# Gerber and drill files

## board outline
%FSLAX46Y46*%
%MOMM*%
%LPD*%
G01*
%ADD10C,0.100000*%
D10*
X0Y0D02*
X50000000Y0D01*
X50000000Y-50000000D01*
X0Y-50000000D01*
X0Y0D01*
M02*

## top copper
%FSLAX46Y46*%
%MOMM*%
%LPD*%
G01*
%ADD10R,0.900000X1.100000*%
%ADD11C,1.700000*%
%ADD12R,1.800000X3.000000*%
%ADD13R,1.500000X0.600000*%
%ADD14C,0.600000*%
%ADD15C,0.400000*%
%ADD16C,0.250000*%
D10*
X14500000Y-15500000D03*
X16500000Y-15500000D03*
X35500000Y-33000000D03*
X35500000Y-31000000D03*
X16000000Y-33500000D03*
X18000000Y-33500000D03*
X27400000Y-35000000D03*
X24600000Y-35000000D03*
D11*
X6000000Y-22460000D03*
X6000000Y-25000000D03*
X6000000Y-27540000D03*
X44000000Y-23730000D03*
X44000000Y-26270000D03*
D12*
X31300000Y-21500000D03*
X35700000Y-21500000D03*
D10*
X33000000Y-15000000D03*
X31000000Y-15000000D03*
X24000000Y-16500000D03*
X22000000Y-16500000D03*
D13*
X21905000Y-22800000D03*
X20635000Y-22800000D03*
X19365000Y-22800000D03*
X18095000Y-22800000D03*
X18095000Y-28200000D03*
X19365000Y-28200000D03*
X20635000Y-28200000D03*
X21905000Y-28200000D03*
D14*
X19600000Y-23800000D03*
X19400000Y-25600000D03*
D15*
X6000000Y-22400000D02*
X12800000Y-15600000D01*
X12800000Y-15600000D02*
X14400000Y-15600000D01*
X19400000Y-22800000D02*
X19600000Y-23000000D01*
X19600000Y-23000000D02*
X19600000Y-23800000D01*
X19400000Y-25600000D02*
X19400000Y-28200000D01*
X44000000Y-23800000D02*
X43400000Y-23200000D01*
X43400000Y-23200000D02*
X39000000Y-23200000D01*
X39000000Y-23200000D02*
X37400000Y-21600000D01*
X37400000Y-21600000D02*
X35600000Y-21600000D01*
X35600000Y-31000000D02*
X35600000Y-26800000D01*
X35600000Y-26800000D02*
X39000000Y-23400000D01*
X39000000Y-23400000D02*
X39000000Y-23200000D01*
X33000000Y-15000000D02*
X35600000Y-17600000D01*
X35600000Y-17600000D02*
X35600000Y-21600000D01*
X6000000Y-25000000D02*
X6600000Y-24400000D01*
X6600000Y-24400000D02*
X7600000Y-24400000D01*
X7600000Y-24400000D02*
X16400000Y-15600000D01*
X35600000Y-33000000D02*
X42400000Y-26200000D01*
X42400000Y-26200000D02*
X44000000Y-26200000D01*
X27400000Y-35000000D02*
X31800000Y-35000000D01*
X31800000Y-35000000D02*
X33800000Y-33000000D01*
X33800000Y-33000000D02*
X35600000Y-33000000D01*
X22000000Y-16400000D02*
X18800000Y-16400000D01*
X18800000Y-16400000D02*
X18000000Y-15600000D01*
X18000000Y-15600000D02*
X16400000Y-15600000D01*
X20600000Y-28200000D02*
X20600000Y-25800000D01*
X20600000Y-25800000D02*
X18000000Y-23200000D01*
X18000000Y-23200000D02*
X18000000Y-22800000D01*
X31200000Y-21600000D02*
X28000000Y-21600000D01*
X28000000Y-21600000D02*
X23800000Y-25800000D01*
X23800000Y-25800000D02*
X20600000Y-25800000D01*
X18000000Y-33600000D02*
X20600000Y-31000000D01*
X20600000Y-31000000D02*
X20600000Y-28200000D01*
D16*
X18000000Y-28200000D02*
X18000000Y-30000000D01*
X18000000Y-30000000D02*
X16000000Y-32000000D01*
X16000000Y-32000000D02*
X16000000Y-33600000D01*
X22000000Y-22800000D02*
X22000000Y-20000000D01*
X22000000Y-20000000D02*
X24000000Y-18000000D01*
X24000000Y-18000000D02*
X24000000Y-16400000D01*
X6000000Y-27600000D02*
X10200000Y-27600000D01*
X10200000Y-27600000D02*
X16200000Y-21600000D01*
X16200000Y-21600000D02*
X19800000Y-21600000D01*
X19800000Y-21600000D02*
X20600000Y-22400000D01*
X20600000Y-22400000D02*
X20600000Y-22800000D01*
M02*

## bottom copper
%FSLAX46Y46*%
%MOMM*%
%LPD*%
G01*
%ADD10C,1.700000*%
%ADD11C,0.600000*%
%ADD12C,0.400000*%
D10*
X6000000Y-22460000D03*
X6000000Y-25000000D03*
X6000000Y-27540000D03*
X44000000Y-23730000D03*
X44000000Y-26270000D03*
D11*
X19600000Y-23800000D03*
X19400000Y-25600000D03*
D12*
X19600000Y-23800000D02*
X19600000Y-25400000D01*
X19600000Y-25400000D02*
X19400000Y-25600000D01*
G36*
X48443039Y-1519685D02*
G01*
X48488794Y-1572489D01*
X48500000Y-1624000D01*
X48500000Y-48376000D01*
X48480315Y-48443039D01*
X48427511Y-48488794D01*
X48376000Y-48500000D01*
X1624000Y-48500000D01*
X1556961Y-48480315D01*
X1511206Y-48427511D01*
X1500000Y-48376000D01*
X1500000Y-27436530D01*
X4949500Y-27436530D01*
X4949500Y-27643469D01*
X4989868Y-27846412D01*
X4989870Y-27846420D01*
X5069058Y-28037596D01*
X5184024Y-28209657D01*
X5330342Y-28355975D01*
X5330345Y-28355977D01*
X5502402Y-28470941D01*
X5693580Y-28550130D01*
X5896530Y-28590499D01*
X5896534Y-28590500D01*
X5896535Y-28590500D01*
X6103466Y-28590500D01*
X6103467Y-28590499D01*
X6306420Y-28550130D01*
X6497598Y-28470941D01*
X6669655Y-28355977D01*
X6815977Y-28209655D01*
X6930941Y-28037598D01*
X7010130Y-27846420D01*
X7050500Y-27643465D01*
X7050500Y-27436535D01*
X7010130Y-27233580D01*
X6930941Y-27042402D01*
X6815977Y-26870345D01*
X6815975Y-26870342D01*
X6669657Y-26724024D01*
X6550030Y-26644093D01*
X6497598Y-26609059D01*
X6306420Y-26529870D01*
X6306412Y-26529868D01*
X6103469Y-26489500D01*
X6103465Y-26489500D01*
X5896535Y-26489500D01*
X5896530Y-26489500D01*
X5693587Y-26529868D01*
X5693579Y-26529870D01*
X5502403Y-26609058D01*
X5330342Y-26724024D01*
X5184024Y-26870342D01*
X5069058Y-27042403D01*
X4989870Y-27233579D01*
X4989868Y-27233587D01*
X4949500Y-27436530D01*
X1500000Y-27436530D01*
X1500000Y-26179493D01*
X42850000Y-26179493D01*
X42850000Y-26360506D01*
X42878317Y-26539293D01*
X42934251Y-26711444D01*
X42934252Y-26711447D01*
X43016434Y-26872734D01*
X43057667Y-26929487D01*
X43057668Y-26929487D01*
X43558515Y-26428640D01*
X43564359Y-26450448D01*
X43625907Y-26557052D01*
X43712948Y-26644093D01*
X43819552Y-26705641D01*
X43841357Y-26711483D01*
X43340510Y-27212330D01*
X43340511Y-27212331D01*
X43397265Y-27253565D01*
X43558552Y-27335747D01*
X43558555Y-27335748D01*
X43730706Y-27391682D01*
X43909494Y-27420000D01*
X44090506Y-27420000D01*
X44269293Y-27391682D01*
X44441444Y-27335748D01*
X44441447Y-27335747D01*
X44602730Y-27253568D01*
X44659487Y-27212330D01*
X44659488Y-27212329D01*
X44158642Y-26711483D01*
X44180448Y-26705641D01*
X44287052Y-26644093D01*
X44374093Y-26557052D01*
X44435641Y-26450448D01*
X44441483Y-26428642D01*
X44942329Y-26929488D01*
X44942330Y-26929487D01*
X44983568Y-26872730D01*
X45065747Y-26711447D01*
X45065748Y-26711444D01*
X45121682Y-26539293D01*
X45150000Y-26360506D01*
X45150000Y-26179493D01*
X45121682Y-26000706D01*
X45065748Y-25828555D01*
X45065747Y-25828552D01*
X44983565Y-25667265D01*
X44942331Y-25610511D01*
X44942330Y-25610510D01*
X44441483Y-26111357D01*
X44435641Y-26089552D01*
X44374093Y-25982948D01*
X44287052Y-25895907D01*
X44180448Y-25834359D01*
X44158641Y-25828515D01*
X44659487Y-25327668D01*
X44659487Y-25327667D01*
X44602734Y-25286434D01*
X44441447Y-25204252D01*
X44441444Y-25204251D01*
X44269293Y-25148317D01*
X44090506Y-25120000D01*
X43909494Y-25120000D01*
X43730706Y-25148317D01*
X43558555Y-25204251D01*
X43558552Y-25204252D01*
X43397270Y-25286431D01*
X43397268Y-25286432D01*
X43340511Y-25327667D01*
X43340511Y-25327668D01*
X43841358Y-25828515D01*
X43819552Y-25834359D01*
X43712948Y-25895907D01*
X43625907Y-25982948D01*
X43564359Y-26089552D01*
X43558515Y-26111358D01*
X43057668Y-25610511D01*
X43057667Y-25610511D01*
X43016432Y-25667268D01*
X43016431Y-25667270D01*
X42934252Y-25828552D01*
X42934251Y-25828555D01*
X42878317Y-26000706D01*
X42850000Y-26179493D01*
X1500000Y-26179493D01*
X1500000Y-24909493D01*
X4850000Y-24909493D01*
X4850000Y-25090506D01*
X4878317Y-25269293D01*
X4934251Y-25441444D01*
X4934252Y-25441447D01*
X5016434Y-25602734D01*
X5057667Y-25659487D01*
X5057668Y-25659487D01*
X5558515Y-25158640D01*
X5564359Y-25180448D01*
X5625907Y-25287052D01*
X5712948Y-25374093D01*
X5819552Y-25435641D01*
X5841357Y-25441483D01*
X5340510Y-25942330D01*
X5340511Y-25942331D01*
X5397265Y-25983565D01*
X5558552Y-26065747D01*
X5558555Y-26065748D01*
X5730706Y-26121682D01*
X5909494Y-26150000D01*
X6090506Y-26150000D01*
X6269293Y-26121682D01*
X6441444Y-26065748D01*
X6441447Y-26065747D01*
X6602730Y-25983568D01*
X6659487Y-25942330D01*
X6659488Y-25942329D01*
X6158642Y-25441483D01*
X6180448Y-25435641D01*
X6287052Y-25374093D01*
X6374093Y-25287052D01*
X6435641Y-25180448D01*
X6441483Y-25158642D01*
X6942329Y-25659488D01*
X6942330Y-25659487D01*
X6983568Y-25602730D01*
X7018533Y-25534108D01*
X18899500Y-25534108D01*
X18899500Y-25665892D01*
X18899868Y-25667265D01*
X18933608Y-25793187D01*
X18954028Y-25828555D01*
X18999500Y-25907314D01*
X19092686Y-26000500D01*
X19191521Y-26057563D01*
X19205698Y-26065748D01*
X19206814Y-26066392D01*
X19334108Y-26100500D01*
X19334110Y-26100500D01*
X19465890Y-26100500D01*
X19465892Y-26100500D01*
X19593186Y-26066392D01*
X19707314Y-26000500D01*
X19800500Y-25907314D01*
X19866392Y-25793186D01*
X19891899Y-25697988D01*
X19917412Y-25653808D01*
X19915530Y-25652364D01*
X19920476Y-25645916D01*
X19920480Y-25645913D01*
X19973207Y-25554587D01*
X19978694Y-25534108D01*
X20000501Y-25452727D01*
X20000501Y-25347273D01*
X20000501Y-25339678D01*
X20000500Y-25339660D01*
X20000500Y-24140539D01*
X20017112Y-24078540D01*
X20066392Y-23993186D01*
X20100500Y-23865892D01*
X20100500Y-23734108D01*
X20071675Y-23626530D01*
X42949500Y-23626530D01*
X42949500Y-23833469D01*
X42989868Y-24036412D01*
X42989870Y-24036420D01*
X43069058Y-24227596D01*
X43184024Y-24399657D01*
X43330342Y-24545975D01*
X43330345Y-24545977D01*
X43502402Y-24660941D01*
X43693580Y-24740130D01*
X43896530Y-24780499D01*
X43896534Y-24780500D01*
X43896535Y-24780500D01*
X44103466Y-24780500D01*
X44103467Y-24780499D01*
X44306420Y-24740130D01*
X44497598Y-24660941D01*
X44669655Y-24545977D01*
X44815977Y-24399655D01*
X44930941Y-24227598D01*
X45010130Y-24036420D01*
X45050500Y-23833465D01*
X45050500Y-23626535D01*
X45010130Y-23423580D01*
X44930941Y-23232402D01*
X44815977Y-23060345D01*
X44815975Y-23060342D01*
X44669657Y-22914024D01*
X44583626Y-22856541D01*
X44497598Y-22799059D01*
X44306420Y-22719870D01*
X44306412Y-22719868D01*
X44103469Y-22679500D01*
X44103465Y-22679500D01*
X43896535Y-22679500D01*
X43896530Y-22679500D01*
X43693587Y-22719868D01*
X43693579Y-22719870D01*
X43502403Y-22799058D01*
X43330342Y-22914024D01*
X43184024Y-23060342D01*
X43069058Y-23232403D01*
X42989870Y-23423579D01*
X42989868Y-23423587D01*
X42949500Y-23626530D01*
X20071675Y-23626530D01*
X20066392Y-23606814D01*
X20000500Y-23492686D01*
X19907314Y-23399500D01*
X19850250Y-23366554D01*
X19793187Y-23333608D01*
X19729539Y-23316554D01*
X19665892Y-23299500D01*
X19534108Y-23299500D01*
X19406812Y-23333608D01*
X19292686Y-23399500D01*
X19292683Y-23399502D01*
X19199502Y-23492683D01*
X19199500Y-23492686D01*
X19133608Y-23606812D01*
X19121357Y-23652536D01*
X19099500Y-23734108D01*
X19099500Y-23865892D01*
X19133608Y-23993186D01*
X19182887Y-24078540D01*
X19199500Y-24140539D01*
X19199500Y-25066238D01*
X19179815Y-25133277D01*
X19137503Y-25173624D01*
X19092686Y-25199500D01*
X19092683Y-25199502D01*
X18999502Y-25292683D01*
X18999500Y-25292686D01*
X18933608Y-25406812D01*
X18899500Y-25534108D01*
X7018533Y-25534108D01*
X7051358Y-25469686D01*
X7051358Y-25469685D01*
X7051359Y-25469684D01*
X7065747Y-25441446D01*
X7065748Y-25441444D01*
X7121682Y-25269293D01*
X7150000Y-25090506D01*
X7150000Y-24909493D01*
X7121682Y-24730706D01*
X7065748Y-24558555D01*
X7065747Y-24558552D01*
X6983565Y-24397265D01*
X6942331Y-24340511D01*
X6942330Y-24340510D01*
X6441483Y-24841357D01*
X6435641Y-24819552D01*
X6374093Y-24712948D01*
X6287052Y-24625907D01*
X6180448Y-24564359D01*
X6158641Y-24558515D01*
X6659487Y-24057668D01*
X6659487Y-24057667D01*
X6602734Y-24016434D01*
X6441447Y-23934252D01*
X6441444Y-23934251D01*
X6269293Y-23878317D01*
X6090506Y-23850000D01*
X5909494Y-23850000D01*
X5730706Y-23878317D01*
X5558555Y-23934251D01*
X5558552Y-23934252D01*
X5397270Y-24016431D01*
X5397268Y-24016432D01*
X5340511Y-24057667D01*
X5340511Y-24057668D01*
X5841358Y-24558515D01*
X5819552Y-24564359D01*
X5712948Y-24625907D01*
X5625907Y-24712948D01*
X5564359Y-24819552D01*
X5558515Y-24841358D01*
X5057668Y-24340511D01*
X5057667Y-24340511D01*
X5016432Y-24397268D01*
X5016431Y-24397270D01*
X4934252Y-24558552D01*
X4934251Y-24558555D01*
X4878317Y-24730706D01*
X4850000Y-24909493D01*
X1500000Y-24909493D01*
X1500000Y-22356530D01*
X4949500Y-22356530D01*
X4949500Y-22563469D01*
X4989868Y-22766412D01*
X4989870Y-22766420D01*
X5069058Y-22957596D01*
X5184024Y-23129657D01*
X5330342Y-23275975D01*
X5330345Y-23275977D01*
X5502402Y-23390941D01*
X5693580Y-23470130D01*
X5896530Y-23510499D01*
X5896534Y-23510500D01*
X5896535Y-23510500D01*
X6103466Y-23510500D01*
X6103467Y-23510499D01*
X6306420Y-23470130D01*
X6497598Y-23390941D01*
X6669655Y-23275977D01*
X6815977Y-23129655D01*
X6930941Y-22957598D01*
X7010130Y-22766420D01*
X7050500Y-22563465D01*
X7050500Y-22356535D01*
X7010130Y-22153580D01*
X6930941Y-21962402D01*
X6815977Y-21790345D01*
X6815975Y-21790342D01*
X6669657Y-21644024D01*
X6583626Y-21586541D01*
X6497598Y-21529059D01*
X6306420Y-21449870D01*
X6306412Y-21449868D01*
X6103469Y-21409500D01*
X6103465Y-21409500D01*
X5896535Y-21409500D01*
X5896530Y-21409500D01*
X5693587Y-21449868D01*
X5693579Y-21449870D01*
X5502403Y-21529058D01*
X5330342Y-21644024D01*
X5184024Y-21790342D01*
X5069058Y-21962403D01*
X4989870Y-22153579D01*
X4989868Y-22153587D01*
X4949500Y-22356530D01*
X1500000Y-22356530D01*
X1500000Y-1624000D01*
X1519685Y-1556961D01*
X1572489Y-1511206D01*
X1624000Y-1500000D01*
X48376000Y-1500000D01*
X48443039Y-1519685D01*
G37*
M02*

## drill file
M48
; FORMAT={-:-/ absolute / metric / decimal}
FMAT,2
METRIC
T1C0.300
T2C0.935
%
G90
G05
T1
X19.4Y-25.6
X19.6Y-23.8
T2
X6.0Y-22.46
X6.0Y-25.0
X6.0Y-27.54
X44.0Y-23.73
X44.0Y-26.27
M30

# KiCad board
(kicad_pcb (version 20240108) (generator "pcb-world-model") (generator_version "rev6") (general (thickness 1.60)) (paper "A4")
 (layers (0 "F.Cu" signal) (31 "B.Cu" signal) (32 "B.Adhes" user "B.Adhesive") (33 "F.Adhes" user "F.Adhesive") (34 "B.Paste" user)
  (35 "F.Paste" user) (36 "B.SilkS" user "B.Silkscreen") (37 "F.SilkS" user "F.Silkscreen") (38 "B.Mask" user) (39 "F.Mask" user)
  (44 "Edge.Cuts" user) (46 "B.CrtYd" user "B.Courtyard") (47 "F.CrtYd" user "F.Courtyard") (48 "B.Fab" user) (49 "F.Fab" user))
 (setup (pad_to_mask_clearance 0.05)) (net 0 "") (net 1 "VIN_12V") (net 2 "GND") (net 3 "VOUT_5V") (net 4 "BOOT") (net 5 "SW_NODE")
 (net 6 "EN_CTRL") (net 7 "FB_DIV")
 (gr_rect (start 0.0 0.0) (end 50.0000 50.0000) (stroke (width 0.1) (type default)) (fill none) (layer "Edge.Cuts"))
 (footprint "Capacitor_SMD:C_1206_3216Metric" (layer "F.Cu") (at 15.5000 15.5000 0)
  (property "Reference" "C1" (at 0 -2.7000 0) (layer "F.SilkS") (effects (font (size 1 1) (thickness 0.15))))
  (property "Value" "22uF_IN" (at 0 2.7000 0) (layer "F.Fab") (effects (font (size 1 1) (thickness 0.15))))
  (pad "1" smd rect (at -1.0000 0.0000) (size 0.9000 1.1000) (layers "F.Cu" "F.Paste" "F.Mask") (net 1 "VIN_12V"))
  (pad "2" smd rect (at 1.0000 0.0000) (size 0.9000 1.1000) (layers "F.Cu" "F.Paste" "F.Mask") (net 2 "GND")))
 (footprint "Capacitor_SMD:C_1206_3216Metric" (layer "F.Cu") (at 35.5000 32.0000 90)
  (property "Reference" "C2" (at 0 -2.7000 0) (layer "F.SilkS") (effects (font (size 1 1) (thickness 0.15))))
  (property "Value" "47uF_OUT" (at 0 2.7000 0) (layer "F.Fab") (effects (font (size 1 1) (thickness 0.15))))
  (pad "1" smd rect (at -1.0000 0.0000) (size 0.9000 1.1000) (layers "F.Cu" "F.Paste" "F.Mask") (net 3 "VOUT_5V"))
  (pad "2" smd rect (at 1.0000 0.0000) (size 0.9000 1.1000) (layers "F.Cu" "F.Paste" "F.Mask") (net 2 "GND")))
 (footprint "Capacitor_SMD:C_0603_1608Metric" (layer "F.Cu") (at 17.0000 33.5000 0)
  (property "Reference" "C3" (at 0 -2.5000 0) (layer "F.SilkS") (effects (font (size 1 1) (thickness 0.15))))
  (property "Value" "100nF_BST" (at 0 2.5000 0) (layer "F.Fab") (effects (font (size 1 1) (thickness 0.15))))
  (pad "1" smd rect (at -1.0000 0.0000) (size 0.9000 1.1000) (layers "F.Cu" "F.Paste" "F.Mask") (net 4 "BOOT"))
  (pad "2" smd rect (at 1.0000 0.0000) (size 0.9000 1.1000) (layers "F.Cu" "F.Paste" "F.Mask") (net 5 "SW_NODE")))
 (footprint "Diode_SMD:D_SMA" (layer "F.Cu") (at 26.0000 35.0000 180)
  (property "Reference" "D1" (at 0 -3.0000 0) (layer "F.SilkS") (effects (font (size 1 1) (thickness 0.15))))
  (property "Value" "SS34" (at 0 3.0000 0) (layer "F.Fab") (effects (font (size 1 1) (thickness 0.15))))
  (pad "1" smd rect (at -1.4000 0.0000) (size 0.9000 1.1000) (layers "F.Cu" "F.Paste" "F.Mask") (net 2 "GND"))
  (pad "2" smd rect (at 1.4000 0.0000) (size 0.9000 1.1000) (layers "F.Cu" "F.Paste" "F.Mask") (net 5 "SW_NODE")))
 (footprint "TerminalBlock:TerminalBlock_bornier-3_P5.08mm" (layer "F.Cu") (at 6.0000 25.0000 0) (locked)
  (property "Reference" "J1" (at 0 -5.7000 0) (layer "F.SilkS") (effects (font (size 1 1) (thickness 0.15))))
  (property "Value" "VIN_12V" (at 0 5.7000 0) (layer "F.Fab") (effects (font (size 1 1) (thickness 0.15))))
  (pad "1" thru_hole circle (at 0.0000 -2.5400) (size 1.7000 1.7000) (drill 0.9350) (layers "*.Cu" "*.Mask") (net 1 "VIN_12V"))
  (pad "2" thru_hole circle (at 0.0000 0.0000) (size 1.7000 1.7000) (drill 0.9350) (layers "*.Cu" "*.Mask") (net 2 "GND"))
  (pad "3" thru_hole circle (at 0.0000 2.5400) (size 1.7000 1.7000) (drill 0.9350) (layers "*.Cu" "*.Mask") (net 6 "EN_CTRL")))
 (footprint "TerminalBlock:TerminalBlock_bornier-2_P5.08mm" (layer "F.Cu") (at 44.0000 25.0000 0) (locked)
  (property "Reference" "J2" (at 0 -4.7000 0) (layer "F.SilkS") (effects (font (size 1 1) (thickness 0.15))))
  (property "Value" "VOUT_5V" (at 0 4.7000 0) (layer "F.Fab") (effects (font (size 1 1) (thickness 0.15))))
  (pad "1" thru_hole circle (at 0.0000 -1.2700) (size 1.7000 1.7000) (drill 0.9350) (layers "*.Cu" "*.Mask") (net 3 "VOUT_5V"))
  (pad "2" thru_hole circle (at 0.0000 1.2700) (size 1.7000 1.7000) (drill 0.9350) (layers "*.Cu" "*.Mask") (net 2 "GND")))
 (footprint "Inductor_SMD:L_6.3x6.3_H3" (layer "F.Cu") (at 33.5000 21.5000 0)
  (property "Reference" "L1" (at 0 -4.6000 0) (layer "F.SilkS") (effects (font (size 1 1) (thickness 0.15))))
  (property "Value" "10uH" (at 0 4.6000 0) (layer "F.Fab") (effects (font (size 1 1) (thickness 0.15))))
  (pad "1" smd rect (at -2.2000 0.0000) (size 1.8000 3.0000) (layers "F.Cu" "F.Paste" "F.Mask") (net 5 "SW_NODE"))
  (pad "2" smd rect (at 2.2000 0.0000) (size 1.8000 3.0000) (layers "F.Cu" "F.Paste" "F.Mask") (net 3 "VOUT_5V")))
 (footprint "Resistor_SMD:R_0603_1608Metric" (layer "F.Cu") (at 32.0000 15.0000 180)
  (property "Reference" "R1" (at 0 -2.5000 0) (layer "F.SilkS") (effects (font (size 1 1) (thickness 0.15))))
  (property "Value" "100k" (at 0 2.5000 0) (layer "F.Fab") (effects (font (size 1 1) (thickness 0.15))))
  (pad "1" smd rect (at -1.0000 0.0000) (size 0.9000 1.1000) (layers "F.Cu" "F.Paste" "F.Mask") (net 3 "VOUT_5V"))
  (pad "2" smd rect (at 1.0000 0.0000) (size 0.9000 1.1000) (layers "F.Cu" "F.Paste" "F.Mask") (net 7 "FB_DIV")))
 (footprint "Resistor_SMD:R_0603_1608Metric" (layer "F.Cu") (at 23.0000 16.5000 180)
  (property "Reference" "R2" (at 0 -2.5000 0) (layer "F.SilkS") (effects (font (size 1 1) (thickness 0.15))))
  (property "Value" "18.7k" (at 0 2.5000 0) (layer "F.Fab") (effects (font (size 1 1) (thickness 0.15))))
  (pad "1" smd rect (at -1.0000 0.0000) (size 0.9000 1.1000) (layers "F.Cu" "F.Paste" "F.Mask") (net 7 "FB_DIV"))
  (pad "2" smd rect (at 1.0000 0.0000) (size 0.9000 1.1000) (layers "F.Cu" "F.Paste" "F.Mask") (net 2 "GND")))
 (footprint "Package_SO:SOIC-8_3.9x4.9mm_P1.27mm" (layer "F.Cu") (at 20.0000 25.5000 270)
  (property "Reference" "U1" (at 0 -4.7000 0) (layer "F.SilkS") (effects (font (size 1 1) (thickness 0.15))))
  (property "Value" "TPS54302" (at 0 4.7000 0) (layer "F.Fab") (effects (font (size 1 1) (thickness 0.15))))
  (pad "1" smd rect (at -2.7000 -1.9050) (size 1.5000 0.6000) (layers "F.Cu" "F.Paste" "F.Mask") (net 4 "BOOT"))
  (pad "2" smd rect (at -2.7000 -0.6350) (size 1.5000 0.6000) (layers "F.Cu" "F.Paste" "F.Mask") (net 1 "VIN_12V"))
  (pad "3" smd rect (at -2.7000 0.6350) (size 1.5000 0.6000) (layers "F.Cu" "F.Paste" "F.Mask") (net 5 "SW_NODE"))
  (pad "4" smd rect (at -2.7000 1.9050) (size 1.5000 0.6000) (layers "F.Cu" "F.Paste" "F.Mask") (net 2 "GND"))
  (pad "5" smd rect (at 2.7000 1.9050) (size 1.5000 0.6000) (layers "F.Cu" "F.Paste" "F.Mask") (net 7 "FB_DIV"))
  (pad "6" smd rect (at 2.7000 0.6350) (size 1.5000 0.6000) (layers "F.Cu" "F.Paste" "F.Mask") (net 6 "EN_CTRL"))
  (pad "7" smd rect (at 2.7000 -0.6350) (size 1.5000 0.6000) (layers "F.Cu" "F.Paste" "F.Mask") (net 1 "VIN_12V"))
  (pad "8" smd rect (at 2.7000 -1.9050) (size 1.5000 0.6000) (layers "F.Cu" "F.Paste" "F.Mask") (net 5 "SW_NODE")))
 (segment (start 6.0000 22.4000) (end 12.8000 15.6000) (width 0.4000) (layer "F.Cu") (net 1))
 (segment (start 12.8000 15.6000) (end 14.4000 15.6000) (width 0.4000) (layer "F.Cu") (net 1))
 (segment (start 19.4000 22.8000) (end 19.6000 23.0000) (width 0.4000) (layer "F.Cu") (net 1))
 (segment (start 19.6000 23.0000) (end 19.6000 23.8000) (width 0.4000) (layer "F.Cu") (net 1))
 (segment (start 19.6000 23.8000) (end 19.6000 25.4000) (width 0.4000) (layer "B.Cu") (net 1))
 (segment (start 19.6000 25.4000) (end 19.4000 25.6000) (width 0.4000) (layer "B.Cu") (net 1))
 (segment (start 19.4000 25.6000) (end 19.4000 28.2000) (width 0.4000) (layer "F.Cu") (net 1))
 (segment (start 44.0000 23.8000) (end 43.4000 23.2000) (width 0.4000) (layer "F.Cu") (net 3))
 (segment (start 43.4000 23.2000) (end 39.0000 23.2000) (width 0.4000) (layer "F.Cu") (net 3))
 (segment (start 39.0000 23.2000) (end 37.4000 21.6000) (width 0.4000) (layer "F.Cu") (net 3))
 (segment (start 37.4000 21.6000) (end 35.6000 21.6000) (width 0.4000) (layer "F.Cu") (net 3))
 (segment (start 35.6000 31.0000) (end 35.6000 26.8000) (width 0.4000) (layer "F.Cu") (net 3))
 (segment (start 35.6000 26.8000) (end 39.0000 23.4000) (width 0.4000) (layer "F.Cu") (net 3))
 (segment (start 39.0000 23.4000) (end 39.0000 23.2000) (width 0.4000) (layer "F.Cu") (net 3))
 (segment (start 33.0000 15.0000) (end 35.6000 17.6000) (width 0.4000) (layer "F.Cu") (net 3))
 (segment (start 35.6000 17.6000) (end 35.6000 21.6000) (width 0.4000) (layer "F.Cu") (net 3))
 (segment (start 6.0000 25.0000) (end 6.6000 24.4000) (width 0.4000) (layer "F.Cu") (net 2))
 (segment (start 6.6000 24.4000) (end 7.6000 24.4000) (width 0.4000) (layer "F.Cu") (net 2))
 (segment (start 7.6000 24.4000) (end 16.4000 15.6000) (width 0.4000) (layer "F.Cu") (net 2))
 (segment (start 35.6000 33.0000) (end 42.4000 26.2000) (width 0.4000) (layer "F.Cu") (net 2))
 (segment (start 42.4000 26.2000) (end 44.0000 26.2000) (width 0.4000) (layer "F.Cu") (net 2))
 (segment (start 27.4000 35.0000) (end 31.8000 35.0000) (width 0.4000) (layer "F.Cu") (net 2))
 (segment (start 31.8000 35.0000) (end 33.8000 33.0000) (width 0.4000) (layer "F.Cu") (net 2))
 (segment (start 33.8000 33.0000) (end 35.6000 33.0000) (width 0.4000) (layer "F.Cu") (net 2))
 (segment (start 22.0000 16.4000) (end 18.8000 16.4000) (width 0.4000) (layer "F.Cu") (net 2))
 (segment (start 18.8000 16.4000) (end 18.0000 15.6000) (width 0.4000) (layer "F.Cu") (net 2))
 (segment (start 18.0000 15.6000) (end 16.4000 15.6000) (width 0.4000) (layer "F.Cu") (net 2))
 (segment (start 20.6000 28.2000) (end 20.6000 25.8000) (width 0.4000) (layer "F.Cu") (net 5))
 (segment (start 20.6000 25.8000) (end 18.0000 23.2000) (width 0.4000) (layer "F.Cu") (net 5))
 (segment (start 18.0000 23.2000) (end 18.0000 22.8000) (width 0.4000) (layer "F.Cu") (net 5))
 (segment (start 31.2000 21.6000) (end 28.0000 21.6000) (width 0.4000) (layer "F.Cu") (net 5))
 (segment (start 28.0000 21.6000) (end 23.8000 25.8000) (width 0.4000) (layer "F.Cu") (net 5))
 (segment (start 23.8000 25.8000) (end 20.6000 25.8000) (width 0.4000) (layer "F.Cu") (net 5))
 (segment (start 18.0000 33.6000) (end 20.6000 31.0000) (width 0.4000) (layer "F.Cu") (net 5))
 (segment (start 20.6000 31.0000) (end 20.6000 28.2000) (width 0.4000) (layer "F.Cu") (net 5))
 (segment (start 18.0000 28.2000) (end 18.0000 30.0000) (width 0.2500) (layer "F.Cu") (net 4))
 (segment (start 18.0000 30.0000) (end 16.0000 32.0000) (width 0.2500) (layer "F.Cu") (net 4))
 (segment (start 16.0000 32.0000) (end 16.0000 33.6000) (width 0.2500) (layer "F.Cu") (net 4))
 (segment (start 22.0000 22.8000) (end 22.0000 20.0000) (width 0.2500) (layer "F.Cu") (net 7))
 (segment (start 22.0000 20.0000) (end 24.0000 18.0000) (width 0.2500) (layer "F.Cu") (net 7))
 (segment (start 24.0000 18.0000) (end 24.0000 16.4000) (width 0.2500) (layer "F.Cu") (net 7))
 (segment (start 6.0000 27.6000) (end 10.2000 27.6000) (width 0.2500) (layer "F.Cu") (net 6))
 (segment (start 10.2000 27.6000) (end 16.2000 21.6000) (width 0.2500) (layer "F.Cu") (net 6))
 (segment (start 16.2000 21.6000) (end 19.8000 21.6000) (width 0.2500) (layer "F.Cu") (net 6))
 (segment (start 19.8000 21.6000) (end 20.6000 22.4000) (width 0.2500) (layer "F.Cu") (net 6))
 (segment (start 20.6000 22.4000) (end 20.6000 22.8000) (width 0.2500) (layer "F.Cu") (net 6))
 (via (at 19.6000 23.8000) (size 0.6000) (drill 0.3000) (layers "F.Cu" "B.Cu") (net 1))
 (via (at 19.4000 25.6000) (size 0.6000) (drill 0.3000) (layers "F.Cu" "B.Cu") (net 1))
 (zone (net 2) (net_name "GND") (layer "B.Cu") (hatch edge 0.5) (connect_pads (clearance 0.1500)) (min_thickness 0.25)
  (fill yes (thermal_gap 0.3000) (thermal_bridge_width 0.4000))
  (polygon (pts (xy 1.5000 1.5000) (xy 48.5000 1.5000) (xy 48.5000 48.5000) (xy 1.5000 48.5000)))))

